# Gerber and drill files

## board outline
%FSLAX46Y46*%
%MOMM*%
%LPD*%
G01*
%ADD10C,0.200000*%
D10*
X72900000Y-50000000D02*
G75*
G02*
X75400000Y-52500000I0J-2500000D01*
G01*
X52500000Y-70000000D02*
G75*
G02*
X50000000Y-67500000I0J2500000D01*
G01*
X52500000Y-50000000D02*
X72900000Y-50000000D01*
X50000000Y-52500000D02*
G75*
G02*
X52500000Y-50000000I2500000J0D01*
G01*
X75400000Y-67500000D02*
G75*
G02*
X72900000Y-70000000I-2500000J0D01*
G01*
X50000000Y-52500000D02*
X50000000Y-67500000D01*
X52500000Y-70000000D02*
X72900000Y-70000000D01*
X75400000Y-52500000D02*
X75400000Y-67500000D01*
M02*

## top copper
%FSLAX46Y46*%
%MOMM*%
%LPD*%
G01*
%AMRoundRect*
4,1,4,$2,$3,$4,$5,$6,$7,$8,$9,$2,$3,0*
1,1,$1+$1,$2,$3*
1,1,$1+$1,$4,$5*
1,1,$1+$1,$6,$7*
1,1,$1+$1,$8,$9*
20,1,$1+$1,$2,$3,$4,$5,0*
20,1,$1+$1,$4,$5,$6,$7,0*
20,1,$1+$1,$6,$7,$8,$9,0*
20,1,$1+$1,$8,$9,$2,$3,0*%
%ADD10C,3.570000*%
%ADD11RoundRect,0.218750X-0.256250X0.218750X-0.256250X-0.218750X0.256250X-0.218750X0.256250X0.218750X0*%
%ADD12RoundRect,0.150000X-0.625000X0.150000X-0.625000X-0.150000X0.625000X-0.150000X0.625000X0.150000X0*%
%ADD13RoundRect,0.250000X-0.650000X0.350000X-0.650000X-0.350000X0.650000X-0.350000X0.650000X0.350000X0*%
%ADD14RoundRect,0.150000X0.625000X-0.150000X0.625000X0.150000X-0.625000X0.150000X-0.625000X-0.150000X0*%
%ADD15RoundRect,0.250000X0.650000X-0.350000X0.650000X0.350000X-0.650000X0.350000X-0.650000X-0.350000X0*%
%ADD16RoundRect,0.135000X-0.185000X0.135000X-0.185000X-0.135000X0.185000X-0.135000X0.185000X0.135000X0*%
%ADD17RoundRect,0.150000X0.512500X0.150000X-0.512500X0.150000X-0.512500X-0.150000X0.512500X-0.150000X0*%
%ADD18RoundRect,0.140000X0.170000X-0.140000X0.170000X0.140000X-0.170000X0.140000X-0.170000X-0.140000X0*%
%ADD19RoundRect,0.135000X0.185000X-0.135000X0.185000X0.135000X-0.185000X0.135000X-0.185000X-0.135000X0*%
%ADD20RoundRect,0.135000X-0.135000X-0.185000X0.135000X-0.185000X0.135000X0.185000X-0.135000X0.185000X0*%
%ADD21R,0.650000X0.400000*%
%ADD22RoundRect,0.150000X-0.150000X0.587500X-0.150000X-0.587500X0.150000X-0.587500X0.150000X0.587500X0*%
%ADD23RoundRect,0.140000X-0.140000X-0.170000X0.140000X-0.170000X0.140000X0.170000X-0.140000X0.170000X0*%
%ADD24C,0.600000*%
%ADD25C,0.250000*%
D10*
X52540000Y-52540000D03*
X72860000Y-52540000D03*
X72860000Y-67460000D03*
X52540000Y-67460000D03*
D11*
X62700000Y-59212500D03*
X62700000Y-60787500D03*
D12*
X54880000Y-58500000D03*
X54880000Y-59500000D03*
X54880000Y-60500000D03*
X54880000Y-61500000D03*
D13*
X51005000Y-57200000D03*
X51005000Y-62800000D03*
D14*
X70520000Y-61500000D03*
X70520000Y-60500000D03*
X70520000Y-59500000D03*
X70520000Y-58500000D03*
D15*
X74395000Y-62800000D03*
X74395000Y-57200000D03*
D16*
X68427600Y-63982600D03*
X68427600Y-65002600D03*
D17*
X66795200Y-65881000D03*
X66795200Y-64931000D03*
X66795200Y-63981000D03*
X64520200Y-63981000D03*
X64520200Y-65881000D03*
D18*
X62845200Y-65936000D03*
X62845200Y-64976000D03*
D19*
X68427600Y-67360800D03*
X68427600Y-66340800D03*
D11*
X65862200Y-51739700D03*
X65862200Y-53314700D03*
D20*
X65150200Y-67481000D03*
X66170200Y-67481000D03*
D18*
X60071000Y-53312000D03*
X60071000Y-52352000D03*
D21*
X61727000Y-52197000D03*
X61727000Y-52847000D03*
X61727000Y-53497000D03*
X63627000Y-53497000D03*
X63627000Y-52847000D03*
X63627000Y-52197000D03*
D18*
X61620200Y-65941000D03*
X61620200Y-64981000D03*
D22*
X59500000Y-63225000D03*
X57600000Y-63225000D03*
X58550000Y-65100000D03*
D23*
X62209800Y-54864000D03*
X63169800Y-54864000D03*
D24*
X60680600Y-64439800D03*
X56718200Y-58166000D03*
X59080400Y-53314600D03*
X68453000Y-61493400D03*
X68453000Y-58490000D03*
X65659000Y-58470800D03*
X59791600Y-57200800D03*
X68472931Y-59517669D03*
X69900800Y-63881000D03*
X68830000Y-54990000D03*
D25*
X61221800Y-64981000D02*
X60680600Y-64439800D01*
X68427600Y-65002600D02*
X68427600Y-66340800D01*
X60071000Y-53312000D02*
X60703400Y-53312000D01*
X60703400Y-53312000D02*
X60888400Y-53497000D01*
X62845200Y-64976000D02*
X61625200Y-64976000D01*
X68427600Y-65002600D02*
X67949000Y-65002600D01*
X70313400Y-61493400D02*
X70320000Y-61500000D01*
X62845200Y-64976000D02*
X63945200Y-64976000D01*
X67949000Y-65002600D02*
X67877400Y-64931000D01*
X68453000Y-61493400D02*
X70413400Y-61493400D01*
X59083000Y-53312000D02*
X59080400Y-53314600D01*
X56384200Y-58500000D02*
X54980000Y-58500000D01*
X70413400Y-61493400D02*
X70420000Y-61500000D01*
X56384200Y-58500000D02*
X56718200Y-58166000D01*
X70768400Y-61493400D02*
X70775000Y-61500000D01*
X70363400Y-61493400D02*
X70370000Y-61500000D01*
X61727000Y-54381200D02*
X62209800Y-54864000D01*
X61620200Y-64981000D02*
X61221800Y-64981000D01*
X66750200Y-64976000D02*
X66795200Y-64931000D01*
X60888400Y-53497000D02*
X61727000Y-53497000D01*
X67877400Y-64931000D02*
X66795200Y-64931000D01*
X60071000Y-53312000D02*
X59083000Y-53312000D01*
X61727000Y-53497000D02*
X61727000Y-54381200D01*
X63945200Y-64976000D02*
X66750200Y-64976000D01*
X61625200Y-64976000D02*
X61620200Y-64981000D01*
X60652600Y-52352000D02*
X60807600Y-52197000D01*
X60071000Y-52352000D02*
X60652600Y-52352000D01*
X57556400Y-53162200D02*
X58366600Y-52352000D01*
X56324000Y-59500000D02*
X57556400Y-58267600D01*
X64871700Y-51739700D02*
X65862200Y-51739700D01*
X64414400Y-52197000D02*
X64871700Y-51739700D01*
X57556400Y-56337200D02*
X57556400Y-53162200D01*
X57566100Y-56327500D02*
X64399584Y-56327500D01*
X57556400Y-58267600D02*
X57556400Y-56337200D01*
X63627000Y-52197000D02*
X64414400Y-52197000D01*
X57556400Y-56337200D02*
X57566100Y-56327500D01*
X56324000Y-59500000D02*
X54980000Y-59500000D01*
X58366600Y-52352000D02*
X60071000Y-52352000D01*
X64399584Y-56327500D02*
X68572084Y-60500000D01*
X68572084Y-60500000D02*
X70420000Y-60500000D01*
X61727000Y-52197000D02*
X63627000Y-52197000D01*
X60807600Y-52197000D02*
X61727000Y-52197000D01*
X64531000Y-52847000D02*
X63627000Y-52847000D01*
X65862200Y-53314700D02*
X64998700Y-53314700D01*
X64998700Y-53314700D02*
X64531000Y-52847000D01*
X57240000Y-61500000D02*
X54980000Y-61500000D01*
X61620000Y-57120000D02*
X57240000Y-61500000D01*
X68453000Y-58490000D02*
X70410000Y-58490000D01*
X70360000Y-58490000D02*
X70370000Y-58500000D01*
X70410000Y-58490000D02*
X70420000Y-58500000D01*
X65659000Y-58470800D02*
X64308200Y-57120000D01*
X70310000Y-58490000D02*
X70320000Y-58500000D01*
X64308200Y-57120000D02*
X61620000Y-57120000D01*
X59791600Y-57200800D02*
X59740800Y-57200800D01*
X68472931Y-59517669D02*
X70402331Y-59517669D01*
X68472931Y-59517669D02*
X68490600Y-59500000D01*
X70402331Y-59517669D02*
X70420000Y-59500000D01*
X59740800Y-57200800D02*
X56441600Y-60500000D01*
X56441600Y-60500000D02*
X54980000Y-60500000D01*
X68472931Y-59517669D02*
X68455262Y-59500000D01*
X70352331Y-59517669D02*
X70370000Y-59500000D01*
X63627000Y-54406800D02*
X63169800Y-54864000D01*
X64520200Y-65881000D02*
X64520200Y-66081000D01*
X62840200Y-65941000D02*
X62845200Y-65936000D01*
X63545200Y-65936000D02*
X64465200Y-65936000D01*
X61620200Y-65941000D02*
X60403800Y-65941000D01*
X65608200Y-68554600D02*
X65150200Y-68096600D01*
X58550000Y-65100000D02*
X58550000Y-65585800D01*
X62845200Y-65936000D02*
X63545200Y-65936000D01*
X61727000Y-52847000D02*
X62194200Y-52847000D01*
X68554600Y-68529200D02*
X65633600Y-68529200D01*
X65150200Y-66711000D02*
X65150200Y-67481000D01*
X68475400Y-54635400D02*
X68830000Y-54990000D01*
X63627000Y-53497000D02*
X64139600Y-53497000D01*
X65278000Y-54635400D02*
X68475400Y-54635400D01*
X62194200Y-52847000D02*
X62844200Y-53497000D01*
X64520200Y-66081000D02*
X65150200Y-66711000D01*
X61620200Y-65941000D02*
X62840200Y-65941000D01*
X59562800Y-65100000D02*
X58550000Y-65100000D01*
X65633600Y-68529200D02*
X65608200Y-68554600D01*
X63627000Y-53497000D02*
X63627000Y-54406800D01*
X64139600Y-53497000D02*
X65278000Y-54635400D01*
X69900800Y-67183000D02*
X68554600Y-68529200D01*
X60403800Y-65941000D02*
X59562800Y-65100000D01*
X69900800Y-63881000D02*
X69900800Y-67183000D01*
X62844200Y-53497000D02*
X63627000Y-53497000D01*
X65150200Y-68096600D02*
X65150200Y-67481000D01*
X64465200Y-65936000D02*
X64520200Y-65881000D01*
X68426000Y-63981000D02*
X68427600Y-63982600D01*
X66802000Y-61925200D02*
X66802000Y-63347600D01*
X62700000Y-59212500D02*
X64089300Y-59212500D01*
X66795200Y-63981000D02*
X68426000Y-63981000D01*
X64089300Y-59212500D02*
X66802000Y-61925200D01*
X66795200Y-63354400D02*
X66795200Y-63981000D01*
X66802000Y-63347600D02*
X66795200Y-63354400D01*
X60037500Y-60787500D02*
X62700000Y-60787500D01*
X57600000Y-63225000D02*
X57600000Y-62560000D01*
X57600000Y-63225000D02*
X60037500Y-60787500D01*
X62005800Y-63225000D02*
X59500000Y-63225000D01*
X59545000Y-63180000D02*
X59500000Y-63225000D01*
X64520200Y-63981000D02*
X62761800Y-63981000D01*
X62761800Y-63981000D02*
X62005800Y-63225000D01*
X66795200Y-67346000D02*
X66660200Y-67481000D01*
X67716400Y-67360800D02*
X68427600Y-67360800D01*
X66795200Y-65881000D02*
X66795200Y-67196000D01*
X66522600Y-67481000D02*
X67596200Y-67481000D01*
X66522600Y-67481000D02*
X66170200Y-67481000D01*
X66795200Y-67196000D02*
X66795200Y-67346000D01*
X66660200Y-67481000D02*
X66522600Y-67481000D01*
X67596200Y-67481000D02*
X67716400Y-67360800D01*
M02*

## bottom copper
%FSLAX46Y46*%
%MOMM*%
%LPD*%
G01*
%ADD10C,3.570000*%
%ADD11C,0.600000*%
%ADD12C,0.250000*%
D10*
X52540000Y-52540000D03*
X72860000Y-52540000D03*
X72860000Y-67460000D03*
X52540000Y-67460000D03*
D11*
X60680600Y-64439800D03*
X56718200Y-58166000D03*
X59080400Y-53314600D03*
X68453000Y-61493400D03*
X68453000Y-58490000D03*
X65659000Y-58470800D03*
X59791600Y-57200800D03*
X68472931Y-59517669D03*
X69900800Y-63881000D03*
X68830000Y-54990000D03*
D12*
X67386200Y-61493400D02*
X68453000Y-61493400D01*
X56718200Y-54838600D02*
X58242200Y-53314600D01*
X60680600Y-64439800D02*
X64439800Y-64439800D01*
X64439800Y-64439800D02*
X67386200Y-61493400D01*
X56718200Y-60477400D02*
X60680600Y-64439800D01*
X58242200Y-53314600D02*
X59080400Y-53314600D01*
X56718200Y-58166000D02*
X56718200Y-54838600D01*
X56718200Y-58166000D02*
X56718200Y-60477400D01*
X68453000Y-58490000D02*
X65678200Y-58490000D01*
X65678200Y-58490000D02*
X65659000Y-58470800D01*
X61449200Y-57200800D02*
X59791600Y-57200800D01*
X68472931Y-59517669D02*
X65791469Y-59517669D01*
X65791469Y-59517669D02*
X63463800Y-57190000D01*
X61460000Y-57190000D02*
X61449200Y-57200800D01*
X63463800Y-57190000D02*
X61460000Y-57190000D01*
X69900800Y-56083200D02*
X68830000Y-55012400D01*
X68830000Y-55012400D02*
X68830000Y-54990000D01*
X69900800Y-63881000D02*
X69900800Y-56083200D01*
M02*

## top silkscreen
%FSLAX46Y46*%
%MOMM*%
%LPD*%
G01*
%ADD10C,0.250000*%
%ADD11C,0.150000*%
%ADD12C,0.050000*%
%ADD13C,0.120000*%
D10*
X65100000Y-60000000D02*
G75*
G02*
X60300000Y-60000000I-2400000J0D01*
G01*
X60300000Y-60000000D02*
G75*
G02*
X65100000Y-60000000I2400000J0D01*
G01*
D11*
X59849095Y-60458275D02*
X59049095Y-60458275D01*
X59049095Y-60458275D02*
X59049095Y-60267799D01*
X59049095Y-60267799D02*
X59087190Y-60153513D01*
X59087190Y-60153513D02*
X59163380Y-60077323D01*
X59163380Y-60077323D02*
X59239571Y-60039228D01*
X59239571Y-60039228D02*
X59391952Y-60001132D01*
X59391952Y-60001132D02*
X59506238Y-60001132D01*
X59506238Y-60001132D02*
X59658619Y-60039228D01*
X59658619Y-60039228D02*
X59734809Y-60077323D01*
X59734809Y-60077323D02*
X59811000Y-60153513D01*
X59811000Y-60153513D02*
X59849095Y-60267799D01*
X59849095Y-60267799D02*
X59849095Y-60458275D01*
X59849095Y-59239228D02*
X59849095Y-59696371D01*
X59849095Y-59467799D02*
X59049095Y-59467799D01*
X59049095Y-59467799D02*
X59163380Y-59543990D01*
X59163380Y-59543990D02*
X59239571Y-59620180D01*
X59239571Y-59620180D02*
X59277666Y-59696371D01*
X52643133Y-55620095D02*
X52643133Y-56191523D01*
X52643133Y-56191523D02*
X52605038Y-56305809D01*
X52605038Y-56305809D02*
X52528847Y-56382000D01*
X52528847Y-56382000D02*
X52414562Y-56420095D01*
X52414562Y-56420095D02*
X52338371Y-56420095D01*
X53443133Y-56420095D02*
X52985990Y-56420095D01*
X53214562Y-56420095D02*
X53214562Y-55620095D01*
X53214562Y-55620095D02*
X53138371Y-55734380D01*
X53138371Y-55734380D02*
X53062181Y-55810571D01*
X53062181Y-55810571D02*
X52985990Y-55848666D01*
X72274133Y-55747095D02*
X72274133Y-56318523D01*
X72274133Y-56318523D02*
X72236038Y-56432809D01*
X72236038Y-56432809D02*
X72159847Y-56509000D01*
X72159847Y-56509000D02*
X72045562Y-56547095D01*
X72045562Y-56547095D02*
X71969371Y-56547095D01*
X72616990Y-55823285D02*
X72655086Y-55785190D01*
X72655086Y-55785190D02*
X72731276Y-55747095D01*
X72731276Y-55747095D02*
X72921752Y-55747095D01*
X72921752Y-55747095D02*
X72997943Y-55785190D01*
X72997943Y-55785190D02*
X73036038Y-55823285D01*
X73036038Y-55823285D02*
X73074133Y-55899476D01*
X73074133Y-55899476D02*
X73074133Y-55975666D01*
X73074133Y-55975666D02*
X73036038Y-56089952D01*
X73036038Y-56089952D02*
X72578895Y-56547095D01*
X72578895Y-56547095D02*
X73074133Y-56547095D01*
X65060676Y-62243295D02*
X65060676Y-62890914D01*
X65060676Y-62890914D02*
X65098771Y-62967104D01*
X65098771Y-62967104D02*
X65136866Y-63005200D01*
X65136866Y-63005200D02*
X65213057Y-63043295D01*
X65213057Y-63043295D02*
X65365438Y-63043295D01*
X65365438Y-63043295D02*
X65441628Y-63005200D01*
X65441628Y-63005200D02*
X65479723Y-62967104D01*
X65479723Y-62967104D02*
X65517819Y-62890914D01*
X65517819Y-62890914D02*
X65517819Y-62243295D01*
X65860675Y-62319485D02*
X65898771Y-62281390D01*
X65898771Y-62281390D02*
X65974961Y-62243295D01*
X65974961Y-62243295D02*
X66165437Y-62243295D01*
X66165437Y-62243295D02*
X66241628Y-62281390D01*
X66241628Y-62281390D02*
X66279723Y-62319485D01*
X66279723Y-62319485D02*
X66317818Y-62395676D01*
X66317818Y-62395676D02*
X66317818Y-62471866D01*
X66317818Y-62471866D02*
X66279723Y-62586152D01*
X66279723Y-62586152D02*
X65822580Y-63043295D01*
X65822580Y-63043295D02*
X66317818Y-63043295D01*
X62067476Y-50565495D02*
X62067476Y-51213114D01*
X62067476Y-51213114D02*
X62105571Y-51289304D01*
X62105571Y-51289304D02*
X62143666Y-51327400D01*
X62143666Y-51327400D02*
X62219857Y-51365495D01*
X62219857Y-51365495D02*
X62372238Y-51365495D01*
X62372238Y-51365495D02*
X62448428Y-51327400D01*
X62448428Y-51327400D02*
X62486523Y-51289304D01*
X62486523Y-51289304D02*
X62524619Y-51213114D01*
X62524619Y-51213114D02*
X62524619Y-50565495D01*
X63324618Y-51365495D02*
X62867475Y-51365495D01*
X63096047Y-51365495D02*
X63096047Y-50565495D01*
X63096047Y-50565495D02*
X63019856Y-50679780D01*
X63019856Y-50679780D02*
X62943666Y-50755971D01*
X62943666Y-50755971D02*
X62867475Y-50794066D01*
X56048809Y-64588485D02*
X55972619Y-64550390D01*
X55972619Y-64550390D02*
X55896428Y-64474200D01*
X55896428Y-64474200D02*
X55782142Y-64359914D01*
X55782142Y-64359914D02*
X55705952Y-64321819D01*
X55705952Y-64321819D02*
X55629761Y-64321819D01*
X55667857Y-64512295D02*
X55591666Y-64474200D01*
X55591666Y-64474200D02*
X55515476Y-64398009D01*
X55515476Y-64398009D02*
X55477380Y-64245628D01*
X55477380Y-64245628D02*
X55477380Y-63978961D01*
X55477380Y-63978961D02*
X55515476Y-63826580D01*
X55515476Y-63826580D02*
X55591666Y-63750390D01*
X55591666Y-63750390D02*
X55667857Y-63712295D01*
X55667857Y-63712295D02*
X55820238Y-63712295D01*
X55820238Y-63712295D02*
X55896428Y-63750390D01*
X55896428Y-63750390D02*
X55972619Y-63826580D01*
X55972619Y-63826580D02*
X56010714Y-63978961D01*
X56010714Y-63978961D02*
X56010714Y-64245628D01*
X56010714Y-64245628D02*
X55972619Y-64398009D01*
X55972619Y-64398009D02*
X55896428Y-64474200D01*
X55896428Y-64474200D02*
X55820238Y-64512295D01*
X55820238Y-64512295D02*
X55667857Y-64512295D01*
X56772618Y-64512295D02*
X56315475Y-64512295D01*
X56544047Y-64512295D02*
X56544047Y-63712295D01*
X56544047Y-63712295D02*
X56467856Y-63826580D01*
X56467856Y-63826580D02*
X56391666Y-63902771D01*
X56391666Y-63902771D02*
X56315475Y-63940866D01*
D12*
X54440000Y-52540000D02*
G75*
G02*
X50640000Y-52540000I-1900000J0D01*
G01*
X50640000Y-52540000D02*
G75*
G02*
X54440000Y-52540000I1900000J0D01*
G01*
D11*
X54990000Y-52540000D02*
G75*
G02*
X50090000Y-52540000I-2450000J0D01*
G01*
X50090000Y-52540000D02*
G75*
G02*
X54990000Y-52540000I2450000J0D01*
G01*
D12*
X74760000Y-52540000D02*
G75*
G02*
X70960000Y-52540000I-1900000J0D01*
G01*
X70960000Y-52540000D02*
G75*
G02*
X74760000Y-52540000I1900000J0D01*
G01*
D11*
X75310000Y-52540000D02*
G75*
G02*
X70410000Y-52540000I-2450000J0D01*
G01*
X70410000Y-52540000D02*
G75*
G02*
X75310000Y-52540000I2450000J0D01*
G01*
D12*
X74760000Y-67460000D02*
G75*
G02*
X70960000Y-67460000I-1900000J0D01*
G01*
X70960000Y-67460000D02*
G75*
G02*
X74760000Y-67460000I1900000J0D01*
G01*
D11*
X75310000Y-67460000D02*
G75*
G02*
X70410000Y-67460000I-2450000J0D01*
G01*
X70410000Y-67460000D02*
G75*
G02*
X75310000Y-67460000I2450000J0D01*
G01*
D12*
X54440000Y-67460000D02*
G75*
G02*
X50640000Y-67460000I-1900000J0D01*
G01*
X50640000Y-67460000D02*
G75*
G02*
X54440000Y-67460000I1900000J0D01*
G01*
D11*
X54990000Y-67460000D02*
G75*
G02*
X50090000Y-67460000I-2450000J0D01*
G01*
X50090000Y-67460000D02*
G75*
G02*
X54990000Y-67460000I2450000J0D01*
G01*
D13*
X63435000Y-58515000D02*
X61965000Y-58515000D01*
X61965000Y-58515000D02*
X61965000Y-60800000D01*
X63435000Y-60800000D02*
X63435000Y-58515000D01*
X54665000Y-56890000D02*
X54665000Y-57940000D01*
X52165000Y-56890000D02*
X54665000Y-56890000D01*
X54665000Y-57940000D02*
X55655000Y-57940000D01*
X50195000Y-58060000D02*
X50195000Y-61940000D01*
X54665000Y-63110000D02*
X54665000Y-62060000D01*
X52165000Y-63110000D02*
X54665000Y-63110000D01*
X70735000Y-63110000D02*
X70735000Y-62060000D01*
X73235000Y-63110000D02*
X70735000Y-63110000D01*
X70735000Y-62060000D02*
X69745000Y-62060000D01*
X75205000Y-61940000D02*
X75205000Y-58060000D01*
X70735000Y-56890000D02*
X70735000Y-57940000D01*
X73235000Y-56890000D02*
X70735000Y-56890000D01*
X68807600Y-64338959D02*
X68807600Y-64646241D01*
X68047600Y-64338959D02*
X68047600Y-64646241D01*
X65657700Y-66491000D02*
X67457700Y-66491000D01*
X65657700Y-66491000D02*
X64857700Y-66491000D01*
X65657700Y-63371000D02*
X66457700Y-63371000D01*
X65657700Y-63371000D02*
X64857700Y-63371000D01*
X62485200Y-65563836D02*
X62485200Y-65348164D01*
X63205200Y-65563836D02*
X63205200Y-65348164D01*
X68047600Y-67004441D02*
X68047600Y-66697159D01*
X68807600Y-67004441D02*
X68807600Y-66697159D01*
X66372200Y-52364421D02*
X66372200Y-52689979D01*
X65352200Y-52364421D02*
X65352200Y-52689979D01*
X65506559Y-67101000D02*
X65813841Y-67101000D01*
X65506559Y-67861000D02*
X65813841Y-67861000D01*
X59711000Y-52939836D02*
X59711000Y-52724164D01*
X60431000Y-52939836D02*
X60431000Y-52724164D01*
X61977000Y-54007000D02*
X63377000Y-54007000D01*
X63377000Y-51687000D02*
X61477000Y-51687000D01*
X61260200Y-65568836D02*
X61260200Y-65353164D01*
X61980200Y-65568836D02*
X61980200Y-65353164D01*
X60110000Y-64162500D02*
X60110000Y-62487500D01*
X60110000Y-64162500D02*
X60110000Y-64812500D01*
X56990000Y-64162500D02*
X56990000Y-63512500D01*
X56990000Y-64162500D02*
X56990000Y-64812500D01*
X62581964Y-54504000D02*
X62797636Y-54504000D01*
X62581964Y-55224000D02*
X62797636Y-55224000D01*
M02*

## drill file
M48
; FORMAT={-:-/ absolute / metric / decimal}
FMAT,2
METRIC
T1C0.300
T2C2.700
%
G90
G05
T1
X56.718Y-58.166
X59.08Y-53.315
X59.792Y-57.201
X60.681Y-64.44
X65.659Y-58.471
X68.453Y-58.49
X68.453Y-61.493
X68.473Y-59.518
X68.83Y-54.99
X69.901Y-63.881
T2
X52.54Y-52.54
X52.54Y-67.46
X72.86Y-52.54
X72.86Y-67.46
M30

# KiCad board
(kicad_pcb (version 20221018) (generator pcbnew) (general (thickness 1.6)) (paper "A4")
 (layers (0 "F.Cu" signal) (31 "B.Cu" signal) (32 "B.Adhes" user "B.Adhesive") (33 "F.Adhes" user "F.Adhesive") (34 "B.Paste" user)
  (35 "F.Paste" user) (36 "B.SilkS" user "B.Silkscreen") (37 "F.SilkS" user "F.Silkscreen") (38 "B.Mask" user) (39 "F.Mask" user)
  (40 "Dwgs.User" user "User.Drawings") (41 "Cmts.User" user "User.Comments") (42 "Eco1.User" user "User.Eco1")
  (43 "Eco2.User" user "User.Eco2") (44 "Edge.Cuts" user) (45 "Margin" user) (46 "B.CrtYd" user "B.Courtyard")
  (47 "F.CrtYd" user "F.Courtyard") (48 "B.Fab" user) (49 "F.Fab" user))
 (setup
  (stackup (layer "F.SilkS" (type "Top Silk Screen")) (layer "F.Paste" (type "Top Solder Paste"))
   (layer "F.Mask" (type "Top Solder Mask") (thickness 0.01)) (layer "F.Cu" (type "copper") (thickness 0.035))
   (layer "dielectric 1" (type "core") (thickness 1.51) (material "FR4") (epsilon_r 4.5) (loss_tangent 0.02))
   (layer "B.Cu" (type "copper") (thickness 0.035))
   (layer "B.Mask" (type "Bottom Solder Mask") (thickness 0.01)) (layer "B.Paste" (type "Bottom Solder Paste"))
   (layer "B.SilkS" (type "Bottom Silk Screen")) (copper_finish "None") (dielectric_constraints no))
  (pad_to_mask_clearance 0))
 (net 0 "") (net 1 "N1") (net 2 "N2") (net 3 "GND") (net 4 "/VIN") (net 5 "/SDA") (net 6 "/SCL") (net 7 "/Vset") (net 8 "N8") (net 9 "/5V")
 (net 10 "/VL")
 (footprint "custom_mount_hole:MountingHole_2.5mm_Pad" (layer "F.Cu") (at 52.54 52.54)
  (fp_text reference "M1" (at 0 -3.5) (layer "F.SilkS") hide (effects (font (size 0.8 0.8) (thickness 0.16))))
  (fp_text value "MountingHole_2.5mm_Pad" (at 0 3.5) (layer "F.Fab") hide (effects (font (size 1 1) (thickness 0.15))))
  (fp_circle (center 0 0) (end 1.9 0) (stroke (width 0.05) (type solid)) (fill none) (layer "F.SilkS"))
  (fp_circle (center 0 0) (end 2.45 0) (stroke (width 0.15) (type solid)) (fill none) (layer "F.SilkS"))
  (pad "~" thru_hole circle (at 0 0) (size 3.57 3.57) (drill 2.7) (layers "*.Cu" "*.Mask")))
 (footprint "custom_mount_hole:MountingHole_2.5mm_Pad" (layer "F.Cu") (at 72.86 52.54)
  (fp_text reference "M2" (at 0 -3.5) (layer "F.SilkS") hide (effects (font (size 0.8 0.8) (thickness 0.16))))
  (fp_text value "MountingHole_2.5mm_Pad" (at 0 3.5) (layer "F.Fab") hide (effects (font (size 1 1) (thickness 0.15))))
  (fp_circle (center 0 0) (end 1.9 0) (stroke (width 0.05) (type solid)) (fill none) (layer "F.SilkS"))
  (fp_circle (center 0 0) (end 2.45 0) (stroke (width 0.15) (type solid)) (fill none) (layer "F.SilkS"))
  (pad "~" thru_hole circle (at 0 0) (size 3.57 3.57) (drill 2.7) (layers "*.Cu" "*.Mask")))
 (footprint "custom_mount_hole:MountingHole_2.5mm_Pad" (layer "F.Cu") (at 72.86 67.46)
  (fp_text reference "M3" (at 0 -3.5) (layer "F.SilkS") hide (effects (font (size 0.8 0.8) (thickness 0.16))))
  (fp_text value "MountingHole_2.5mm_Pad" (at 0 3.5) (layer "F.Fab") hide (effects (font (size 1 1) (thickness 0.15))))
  (fp_circle (center 0 0) (end 1.9 0) (stroke (width 0.05) (type solid)) (fill none) (layer "F.SilkS"))
  (fp_circle (center 0 0) (end 2.45 0) (stroke (width 0.15) (type solid)) (fill none) (layer "F.SilkS"))
  (pad "~" thru_hole circle (at 0 0) (size 3.57 3.57) (drill 2.7) (layers "*.Cu" "*.Mask")))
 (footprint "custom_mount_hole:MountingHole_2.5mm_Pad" (layer "F.Cu") (at 52.54 67.46)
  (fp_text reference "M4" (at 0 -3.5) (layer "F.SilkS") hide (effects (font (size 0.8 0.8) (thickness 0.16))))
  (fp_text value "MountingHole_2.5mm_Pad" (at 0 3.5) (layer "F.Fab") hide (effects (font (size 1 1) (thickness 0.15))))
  (fp_circle (center 0 0) (end 1.9 0) (stroke (width 0.05) (type solid)) (fill none) (layer "F.SilkS"))
  (fp_circle (center 0 0) (end 2.45 0) (stroke (width 0.15) (type solid)) (fill none) (layer "F.SilkS"))
  (pad "~" thru_hole circle (at 0 0) (size 3.57 3.57) (drill 2.7) (layers "*.Cu" "*.Mask")))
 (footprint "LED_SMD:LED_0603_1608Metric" (layer "F.Cu") (at 62.7 60 -90)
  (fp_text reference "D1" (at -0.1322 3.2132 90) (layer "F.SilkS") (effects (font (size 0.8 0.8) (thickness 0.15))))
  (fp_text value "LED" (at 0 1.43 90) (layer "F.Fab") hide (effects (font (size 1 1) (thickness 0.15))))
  (fp_line (start -1.485 -0.735) (end -1.485 0.735) (stroke (width 0.12) (type solid)) (layer "F.SilkS"))
  (fp_line (start -1.485 0.735) (end 0.8 0.735) (stroke (width 0.12) (type solid)) (layer "F.SilkS"))
  (fp_line (start 0.8 -0.735) (end -1.485 -0.735) (stroke (width 0.12) (type solid)) (layer "F.SilkS"))
  (pad "1" smd roundrect (at -0.7875 0 270) (size 0.875 0.95) (layers "F.Cu" "F.Paste" "F.Mask") (roundrect_rratio 0.25) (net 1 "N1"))
  (pad "2" smd roundrect (at 0.7875 0 270) (size 0.875 0.95) (layers "F.Cu" "F.Paste" "F.Mask") (roundrect_rratio 0.25) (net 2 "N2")))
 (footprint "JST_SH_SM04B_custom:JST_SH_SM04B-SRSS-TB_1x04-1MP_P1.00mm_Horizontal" (layer "F.Cu") (at 52.88 60 -90)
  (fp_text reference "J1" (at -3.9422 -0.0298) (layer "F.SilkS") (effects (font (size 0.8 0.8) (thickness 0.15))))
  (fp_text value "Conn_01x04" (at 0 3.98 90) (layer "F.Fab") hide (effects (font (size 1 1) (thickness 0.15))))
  (fp_line (start -3.11 -1.785) (end -2.06 -1.785) (stroke (width 0.12) (type solid)) (layer "F.SilkS"))
  (fp_line (start -3.11 0.715) (end -3.11 -1.785) (stroke (width 0.12) (type solid)) (layer "F.SilkS"))
  (fp_line (start -2.06 -1.785) (end -2.06 -2.775) (stroke (width 0.12) (type solid)) (layer "F.SilkS"))
  (fp_line (start -1.94 2.685) (end 1.94 2.685) (stroke (width 0.12) (type solid)) (layer "F.SilkS"))
  (fp_line (start 3.11 -1.785) (end 2.06 -1.785) (stroke (width 0.12) (type solid)) (layer "F.SilkS"))
  (fp_line (start 3.11 0.715) (end 3.11 -1.785) (stroke (width 0.12) (type solid)) (layer "F.SilkS"))
  (pad "1" smd roundrect (at -1.5 -2 270) (size 0.6 1.55) (layers "F.Cu" "F.Paste" "F.Mask") (roundrect_rratio 0.25) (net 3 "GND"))
  (pad "2" smd roundrect (at -0.5 -2 270) (size 0.6 1.55) (layers "F.Cu" "F.Paste" "F.Mask") (roundrect_rratio 0.25) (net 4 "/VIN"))
  (pad "3" smd roundrect (at 0.5 -2 270) (size 0.6 1.55) (layers "F.Cu" "F.Paste" "F.Mask") (roundrect_rratio 0.25) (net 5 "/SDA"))
  (pad "4" smd roundrect (at 1.5 -2 270) (size 0.6 1.55) (layers "F.Cu" "F.Paste" "F.Mask") (roundrect_rratio 0.25) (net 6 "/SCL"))
  (pad "MP" smd roundrect (at -2.8 1.875 270) (size 1.2 1.8) (layers "F.Cu" "F.Paste" "F.Mask") (roundrect_rratio 0.2083333333))
  (pad "MP" smd roundrect (at 2.8 1.875 270) (size 1.2 1.8) (layers "F.Cu" "F.Paste" "F.Mask") (roundrect_rratio 0.2083333333)))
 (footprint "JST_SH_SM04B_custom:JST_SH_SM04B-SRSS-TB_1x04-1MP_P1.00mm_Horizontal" (layer "F.Cu") (at 72.52 60 90)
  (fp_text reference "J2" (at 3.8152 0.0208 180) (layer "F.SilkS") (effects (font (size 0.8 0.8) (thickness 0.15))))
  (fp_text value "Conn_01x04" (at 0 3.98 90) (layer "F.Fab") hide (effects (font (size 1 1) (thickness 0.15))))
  (fp_line (start -3.11 -1.785) (end -2.06 -1.785) (stroke (width 0.12) (type solid)) (layer "F.SilkS"))
  (fp_line (start -3.11 0.715) (end -3.11 -1.785) (stroke (width 0.12) (type solid)) (layer "F.SilkS"))
  (fp_line (start -2.06 -1.785) (end -2.06 -2.775) (stroke (width 0.12) (type solid)) (layer "F.SilkS"))
  (fp_line (start -1.94 2.685) (end 1.94 2.685) (stroke (width 0.12) (type solid)) (layer "F.SilkS"))
  (fp_line (start 3.11 -1.785) (end 2.06 -1.785) (stroke (width 0.12) (type solid)) (layer "F.SilkS"))
  (fp_line (start 3.11 0.715) (end 3.11 -1.785) (stroke (width 0.12) (type solid)) (layer "F.SilkS"))
  (pad "1" smd roundrect (at -1.5 -2 90) (size 0.6 1.55) (layers "F.Cu" "F.Paste" "F.Mask") (roundrect_rratio 0.25) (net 3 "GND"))
  (pad "2" smd roundrect (at -0.5 -2 90) (size 0.6 1.55) (layers "F.Cu" "F.Paste" "F.Mask") (roundrect_rratio 0.25) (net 4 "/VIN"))
  (pad "3" smd roundrect (at 0.5 -2 90) (size 0.6 1.55) (layers "F.Cu" "F.Paste" "F.Mask") (roundrect_rratio 0.25) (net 5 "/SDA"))
  (pad "4" smd roundrect (at 1.5 -2 90) (size 0.6 1.55) (layers "F.Cu" "F.Paste" "F.Mask") (roundrect_rratio 0.25) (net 6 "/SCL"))
  (pad "MP" smd roundrect (at -2.8 1.875 90) (size 1.2 1.8) (layers "F.Cu" "F.Paste" "F.Mask") (roundrect_rratio 0.2083333333))
  (pad "MP" smd roundrect (at 2.8 1.875 90) (size 1.2 1.8) (layers "F.Cu" "F.Paste" "F.Mask") (roundrect_rratio 0.2083333333)))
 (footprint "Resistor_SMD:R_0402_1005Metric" (layer "F.Cu") (at 68.4276 64.4926 -90)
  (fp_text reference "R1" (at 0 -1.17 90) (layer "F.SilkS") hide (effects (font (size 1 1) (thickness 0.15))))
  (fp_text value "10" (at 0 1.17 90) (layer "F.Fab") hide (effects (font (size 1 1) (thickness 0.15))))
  (fp_line (start -0.153641 -0.38) (end 0.153641 -0.38) (stroke (width 0.12) (type solid)) (layer "F.SilkS"))
  (fp_line (start -0.153641 0.38) (end 0.153641 0.38) (stroke (width 0.12) (type solid)) (layer "F.SilkS"))
  (pad "1" smd roundrect (at -0.51 0 270) (size 0.54 0.64) (layers "F.Cu" "F.Paste" "F.Mask") (roundrect_rratio 0.25) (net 1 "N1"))
  (pad "2" smd roundrect (at 0.51 0 270) (size 0.54 0.64) (layers "F.Cu" "F.Paste" "F.Mask") (roundrect_rratio 0.25) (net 3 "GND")))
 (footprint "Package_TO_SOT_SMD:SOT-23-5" (layer "F.Cu") (at 65.6577 64.931 180)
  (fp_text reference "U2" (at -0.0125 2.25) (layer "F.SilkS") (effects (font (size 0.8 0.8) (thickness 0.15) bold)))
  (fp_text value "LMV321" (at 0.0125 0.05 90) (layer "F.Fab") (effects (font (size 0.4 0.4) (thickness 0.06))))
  (fp_line (start 0 -1.56) (end -1.8 -1.56) (stroke (width 0.12) (type solid)) (layer "F.SilkS"))
  (fp_line (start 0 -1.56) (end 0.8 -1.56) (stroke (width 0.12) (type solid)) (layer "F.SilkS"))
  (fp_line (start 0 1.56) (end -0.8 1.56) (stroke (width 0.12) (type solid)) (layer "F.SilkS"))
  (fp_line (start 0 1.56) (end 0.8 1.56) (stroke (width 0.12) (type solid)) (layer "F.SilkS"))
  (pad "1" smd roundrect (at -1.1375 -0.95 180) (size 1.325 0.6) (layers "F.Cu" "F.Paste" "F.Mask") (roundrect_rratio 0.25) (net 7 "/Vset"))
  (pad "2" smd roundrect (at -1.1375 0 180) (size 1.325 0.6) (layers "F.Cu" "F.Paste" "F.Mask") (roundrect_rratio 0.25) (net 3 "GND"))
  (pad "3" smd roundrect (at -1.1375 0.95 180) (size 1.325 0.6) (layers "F.Cu" "F.Paste" "F.Mask") (roundrect_rratio 0.25) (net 1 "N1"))
  (pad "4" smd roundrect (at 1.1375 0.95 180) (size 1.325 0.6) (layers "F.Cu" "F.Paste" "F.Mask") (roundrect_rratio 0.25) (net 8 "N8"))
  (pad "5" smd roundrect (at 1.1375 -0.95 180) (size 1.325 0.6) (layers "F.Cu" "F.Paste" "F.Mask") (roundrect_rratio 0.25) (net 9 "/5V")))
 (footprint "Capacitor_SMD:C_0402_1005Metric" (layer "F.Cu") (at 62.8452 65.456 90)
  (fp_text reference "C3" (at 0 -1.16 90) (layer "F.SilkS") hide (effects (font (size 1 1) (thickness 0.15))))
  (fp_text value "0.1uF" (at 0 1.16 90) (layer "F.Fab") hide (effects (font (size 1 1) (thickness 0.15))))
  (fp_line (start -0.107836 -0.36) (end 0.107836 -0.36) (stroke (width 0.12) (type solid)) (layer "F.SilkS"))
  (fp_line (start -0.107836 0.36) (end 0.107836 0.36) (stroke (width 0.12) (type solid)) (layer "F.SilkS"))
  (pad "1" smd roundrect (at -0.48 0 90) (size 0.56 0.62) (layers "F.Cu" "F.Paste" "F.Mask") (roundrect_rratio 0.25) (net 9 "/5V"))
  (pad "2" smd roundrect (at 0.48 0 90) (size 0.56 0.62) (layers "F.Cu" "F.Paste" "F.Mask") (roundrect_rratio 0.25) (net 3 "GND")))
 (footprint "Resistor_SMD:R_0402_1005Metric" (layer "F.Cu") (at 68.4276 66.8508 90)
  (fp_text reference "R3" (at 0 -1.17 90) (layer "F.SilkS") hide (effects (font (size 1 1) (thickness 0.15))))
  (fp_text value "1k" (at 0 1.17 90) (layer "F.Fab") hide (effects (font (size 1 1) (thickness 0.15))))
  (fp_line (start -0.153641 -0.38) (end 0.153641 -0.38) (stroke (width 0.12) (type solid)) (layer "F.SilkS"))
  (fp_line (start -0.153641 0.38) (end 0.153641 0.38) (stroke (width 0.12) (type solid)) (layer "F.SilkS"))
  (pad "1" smd roundrect (at -0.51 0 90) (size 0.54 0.64) (layers "F.Cu" "F.Paste" "F.Mask") (roundrect_rratio 0.25) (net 7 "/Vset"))
  (pad "2" smd roundrect (at 0.51 0 90) (size 0.54 0.64) (layers "F.Cu" "F.Paste" "F.Mask") (roundrect_rratio 0.25) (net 3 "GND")))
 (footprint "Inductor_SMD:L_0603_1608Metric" (layer "F.Cu") (at 65.8622 52.5272 -90)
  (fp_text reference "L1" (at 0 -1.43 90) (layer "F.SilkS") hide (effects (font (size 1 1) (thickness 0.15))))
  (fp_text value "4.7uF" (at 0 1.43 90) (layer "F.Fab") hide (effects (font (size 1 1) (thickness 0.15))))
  (fp_line (start -0.162779 -0.51) (end 0.162779 -0.51) (stroke (width 0.12) (type solid)) (layer "F.SilkS"))
  (fp_line (start -0.162779 0.51) (end 0.162779 0.51) (stroke (width 0.12) (type solid)) (layer "F.SilkS"))
  (pad "1" smd roundrect (at -0.7875 0 270) (size 0.875 0.95) (layers "F.Cu" "F.Paste" "F.Mask") (roundrect_rratio 0.25) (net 4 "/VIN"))
  (pad "2" smd roundrect (at 0.7875 0 270) (size 0.875 0.95) (layers "F.Cu" "F.Paste" "F.Mask") (roundrect_rratio 0.25) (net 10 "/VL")))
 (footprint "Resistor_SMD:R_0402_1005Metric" (layer "F.Cu") (at 65.6602 67.481)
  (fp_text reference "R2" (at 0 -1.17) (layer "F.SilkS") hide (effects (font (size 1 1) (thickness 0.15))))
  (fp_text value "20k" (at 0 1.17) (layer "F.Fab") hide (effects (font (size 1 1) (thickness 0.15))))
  (fp_line (start -0.153641 -0.38) (end 0.153641 -0.38) (stroke (width 0.12) (type solid)) (layer "F.SilkS"))
  (fp_line (start -0.153641 0.38) (end 0.153641 0.38) (stroke (width 0.12) (type solid)) (layer "F.SilkS"))
  (pad "1" smd roundrect (at -0.51 0) (size 0.54 0.64) (layers "F.Cu" "F.Paste" "F.Mask") (roundrect_rratio 0.25) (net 9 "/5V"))
  (pad "2" smd roundrect (at 0.51 0) (size 0.54 0.64) (layers "F.Cu" "F.Paste" "F.Mask") (roundrect_rratio 0.25) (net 7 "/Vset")))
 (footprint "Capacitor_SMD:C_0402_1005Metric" (layer "F.Cu") (at 60.071 52.832 90)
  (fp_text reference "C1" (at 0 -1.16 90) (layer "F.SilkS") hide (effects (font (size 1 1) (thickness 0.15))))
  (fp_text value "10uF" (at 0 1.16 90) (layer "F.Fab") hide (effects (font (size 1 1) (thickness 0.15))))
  (fp_line (start -0.107836 -0.36) (end 0.107836 -0.36) (stroke (width 0.12) (type solid)) (layer "F.SilkS"))
  (fp_line (start -0.107836 0.36) (end 0.107836 0.36) (stroke (width 0.12) (type solid)) (layer "F.SilkS"))
  (pad "1" smd roundrect (at -0.48 0 90) (size 0.56 0.62) (layers "F.Cu" "F.Paste" "F.Mask") (roundrect_rratio 0.25) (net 3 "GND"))
  (pad "2" smd roundrect (at 0.48 0 90) (size 0.56 0.62) (layers "F.Cu" "F.Paste" "F.Mask") (roundrect_rratio 0.25) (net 4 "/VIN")))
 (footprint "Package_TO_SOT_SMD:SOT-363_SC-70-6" (layer "F.Cu") (at 62.677 52.847)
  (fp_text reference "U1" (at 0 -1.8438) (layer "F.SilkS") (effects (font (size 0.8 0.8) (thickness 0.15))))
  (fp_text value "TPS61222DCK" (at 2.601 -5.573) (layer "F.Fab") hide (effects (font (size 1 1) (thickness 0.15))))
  (fp_line (start -0.7 1.16) (end 0.7 1.16) (stroke (width 0.12) (type solid)) (layer "F.SilkS"))
  (fp_line (start 0.7 -1.16) (end -1.2 -1.16) (stroke (width 0.12) (type solid)) (layer "F.SilkS"))
  (pad "1" smd rect (at -0.95 -0.65) (size 0.65 0.4) (layers "F.Cu" "F.Paste" "F.Mask") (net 4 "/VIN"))
  (pad "2" smd rect (at -0.95 0) (size 0.65 0.4) (layers "F.Cu" "F.Paste" "F.Mask") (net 9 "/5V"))
  (pad "3" smd rect (at -0.95 0.65) (size 0.65 0.4) (layers "F.Cu" "F.Paste" "F.Mask") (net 3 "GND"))
  (pad "4" smd rect (at 0.95 0.65) (size 0.65 0.4) (layers "F.Cu" "F.Paste" "F.Mask") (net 9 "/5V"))
  (pad "5" smd rect (at 0.95 0) (size 0.65 0.4) (layers "F.Cu" "F.Paste" "F.Mask") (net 10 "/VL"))
  (pad "6" smd rect (at 0.95 -0.65) (size 0.65 0.4) (layers "F.Cu" "F.Paste" "F.Mask") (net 4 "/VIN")))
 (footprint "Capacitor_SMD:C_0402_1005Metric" (layer "F.Cu") (at 61.6202 65.461 90)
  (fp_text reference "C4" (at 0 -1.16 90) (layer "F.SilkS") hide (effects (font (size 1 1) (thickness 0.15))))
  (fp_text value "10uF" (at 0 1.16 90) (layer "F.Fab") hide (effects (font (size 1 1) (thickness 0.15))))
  (fp_line (start -0.107836 -0.36) (end 0.107836 -0.36) (stroke (width 0.12) (type solid)) (layer "F.SilkS"))
  (fp_line (start -0.107836 0.36) (end 0.107836 0.36) (stroke (width 0.12) (type solid)) (layer "F.SilkS"))
  (pad "1" smd roundrect (at -0.48 0 90) (size 0.56 0.62) (layers "F.Cu" "F.Paste" "F.Mask") (roundrect_rratio 0.25) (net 9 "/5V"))
  (pad "2" smd roundrect (at 0.48 0 90) (size 0.56 0.62) (layers "F.Cu" "F.Paste" "F.Mask") (roundrect_rratio 0.25) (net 3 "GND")))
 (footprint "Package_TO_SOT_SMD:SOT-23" (layer "F.Cu") (at 58.55 64.1625 -90)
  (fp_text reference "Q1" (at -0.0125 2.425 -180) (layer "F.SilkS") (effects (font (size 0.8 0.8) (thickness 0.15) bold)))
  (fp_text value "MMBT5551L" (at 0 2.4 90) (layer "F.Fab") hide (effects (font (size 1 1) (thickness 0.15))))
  (fp_line (start 0 -1.56) (end -1.675 -1.56) (stroke (width 0.12) (type solid)) (layer "F.SilkS"))
  (fp_line (start 0 -1.56) (end 0.65 -1.56) (stroke (width 0.12) (type solid)) (layer "F.SilkS"))
  (fp_line (start 0 1.56) (end -0.65 1.56) (stroke (width 0.12) (type solid)) (layer "F.SilkS"))
  (fp_line (start 0 1.56) (end 0.65 1.56) (stroke (width 0.12) (type solid)) (layer "F.SilkS"))
  (pad "1" smd roundrect (at -0.9375 -0.95 270) (size 1.475 0.6) (layers "F.Cu" "F.Paste" "F.Mask") (roundrect_rratio 0.25) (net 8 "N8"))
  (pad "2" smd roundrect (at -0.9375 0.95 270) (size 1.475 0.6) (layers "F.Cu" "F.Paste" "F.Mask") (roundrect_rratio 0.25) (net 2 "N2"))
  (pad "3" smd roundrect (at 0.9375 0 270) (size 1.475 0.6) (layers "F.Cu" "F.Paste" "F.Mask") (roundrect_rratio 0.25) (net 9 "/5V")))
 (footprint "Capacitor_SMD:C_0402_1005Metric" (layer "F.Cu") (at 62.6898 54.864)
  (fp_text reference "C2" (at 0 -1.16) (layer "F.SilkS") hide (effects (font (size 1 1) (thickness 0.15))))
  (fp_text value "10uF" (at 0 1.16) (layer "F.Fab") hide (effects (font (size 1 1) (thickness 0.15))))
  (fp_line (start -0.107836 -0.36) (end 0.107836 -0.36) (stroke (width 0.12) (type solid)) (layer "F.SilkS"))
  (fp_line (start -0.107836 0.36) (end 0.107836 0.36) (stroke (width 0.12) (type solid)) (layer "F.SilkS"))
  (pad "1" smd roundrect (at -0.48 0) (size 0.56 0.62) (layers "F.Cu" "F.Paste" "F.Mask") (roundrect_rratio 0.25) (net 3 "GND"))
  (pad "2" smd roundrect (at 0.48 0) (size 0.56 0.62) (layers "F.Cu" "F.Paste" "F.Mask") (roundrect_rratio 0.25) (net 9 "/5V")))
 (gr_circle (center 62.7 60) (end 65.1 60) (stroke (width 0.25) (type solid)) (fill none) (layer "F.SilkS"))
 (gr_arc (start 72.9 50) (mid 74.667767 50.732233) (end 75.4 52.5) (stroke (width 0.2) (type solid)) (layer "Edge.Cuts"))
 (gr_arc (start 52.5 70) (mid 50.732233 69.267767) (end 50 67.5) (stroke (width 0.2) (type solid)) (layer "Edge.Cuts"))
 (gr_line (start 52.5 50) (end 72.9 50) (stroke (width 0.2) (type solid)) (layer "Edge.Cuts"))
 (gr_arc (start 50 52.5) (mid 50.732233 50.732233) (end 52.5 50) (stroke (width 0.2) (type solid)) (layer "Edge.Cuts"))
 (gr_arc (start 75.4 67.5) (mid 74.667767 69.267767) (end 72.9 70) (stroke (width 0.2) (type solid)) (layer "Edge.Cuts"))
 (gr_line (start 50 52.5) (end 50 67.5) (stroke (width 0.2) (type solid)) (layer "Edge.Cuts"))
 (gr_line (start 52.5 70) (end 72.9 70) (stroke (width 0.2) (type solid)) (layer "Edge.Cuts"))
 (gr_line (start 75.4 52.5) (end 75.4 67.5) (stroke (width 0.2) (type solid)) (layer "Edge.Cuts"))
 (segment (start 61.2218 64.981) (end 60.6806 64.4398) (width 0.25) (layer "F.Cu") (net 3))
 (segment (start 68.4276 65.0026) (end 68.4276 66.3408) (width 0.25) (layer "F.Cu") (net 3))
 (segment (start 60.071 53.312) (end 60.7034 53.312) (width 0.25) (layer "F.Cu") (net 3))
 (segment (start 60.7034 53.312) (end 60.8884 53.497) (width 0.25) (layer "F.Cu") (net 3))
 (segment (start 62.8452 64.976) (end 61.6252 64.976) (width 0.25) (layer "F.Cu") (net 3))
 (segment (start 68.4276 65.0026) (end 67.949 65.0026) (width 0.25) (layer "F.Cu") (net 3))
 (segment (start 70.3134 61.4934) (end 70.32 61.5) (width 0.25) (layer "F.Cu") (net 3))
 (segment (start 62.8452 64.976) (end 63.9452 64.976) (width 0.25) (layer "F.Cu") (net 3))
 (segment (start 67.949 65.0026) (end 67.8774 64.931) (width 0.25) (layer "F.Cu") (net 3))
 (segment (start 68.453 61.4934) (end 70.4134 61.4934) (width 0.25) (layer "F.Cu") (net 3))
 (segment (start 59.083 53.312) (end 59.0804 53.3146) (width 0.25) (layer "F.Cu") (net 3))
 (segment (start 56.3842 58.5) (end 54.98 58.5) (width 0.25) (layer "F.Cu") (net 3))
 (segment (start 70.4134 61.4934) (end 70.42 61.5) (width 0.25) (layer "F.Cu") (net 3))
 (segment (start 56.3842 58.5) (end 56.7182 58.166) (width 0.25) (layer "F.Cu") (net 3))
 (segment (start 70.7684 61.4934) (end 70.775 61.5) (width 0.25) (layer "F.Cu") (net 3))
 (segment (start 70.3634 61.4934) (end 70.37 61.5) (width 0.25) (layer "F.Cu") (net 3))
 (segment (start 61.727 54.3812) (end 62.2098 54.864) (width 0.25) (layer "F.Cu") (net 3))
 (segment (start 61.6202 64.981) (end 61.2218 64.981) (width 0.25) (layer "F.Cu") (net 3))
 (segment (start 66.7502 64.976) (end 66.7952 64.931) (width 0.25) (layer "F.Cu") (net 3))
 (segment (start 60.8884 53.497) (end 61.727 53.497) (width 0.25) (layer "F.Cu") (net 3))
 (segment (start 67.8774 64.931) (end 66.7952 64.931) (width 0.25) (layer "F.Cu") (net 3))
 (segment (start 60.071 53.312) (end 59.083 53.312) (width 0.25) (layer "F.Cu") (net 3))
 (segment (start 61.727 53.497) (end 61.727 54.3812) (width 0.25) (layer "F.Cu") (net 3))
 (segment (start 63.9452 64.976) (end 66.7502 64.976) (width 0.25) (layer "F.Cu") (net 3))
 (segment (start 61.6252 64.976) (end 61.6202 64.981) (width 0.25) (layer "F.Cu") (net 3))
 (via (at 60.6806 64.4398) (size 0.6) (drill 0.3) (layers "F.Cu" "B.Cu") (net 3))
 (via (at 56.7182 58.166) (size 0.6) (drill 0.3) (layers "F.Cu" "B.Cu") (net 3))
 (via (at 59.0804 53.3146) (size 0.6) (drill 0.3) (layers "F.Cu" "B.Cu") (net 3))
 (via (at 68.453 61.4934) (size 0.6) (drill 0.3) (layers "F.Cu" "B.Cu") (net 3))
 (segment (start 67.3862 61.4934) (end 68.453 61.4934) (width 0.25) (layer "B.Cu") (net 3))
 (segment (start 56.7182 54.8386) (end 58.2422 53.3146) (width 0.25) (layer "B.Cu") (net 3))
 (segment (start 60.6806 64.4398) (end 64.4398 64.4398) (width 0.25) (layer "B.Cu") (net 3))
 (segment (start 64.4398 64.4398) (end 67.3862 61.4934) (width 0.25) (layer "B.Cu") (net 3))
 (segment (start 56.7182 60.4774) (end 60.6806 64.4398) (width 0.25) (layer "B.Cu") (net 3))
 (segment (start 58.2422 53.3146) (end 59.0804 53.3146) (width 0.25) (layer "B.Cu") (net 3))
 (segment (start 56.7182 58.166) (end 56.7182 54.8386) (width 0.25) (layer "B.Cu") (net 3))
 (segment (start 56.7182 58.166) (end 56.7182 60.4774) (width 0.25) (layer "B.Cu") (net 3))
 (segment (start 60.6526 52.352) (end 60.8076 52.197) (width 0.25) (layer "F.Cu") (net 4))
 (segment (start 60.071 52.352) (end 60.6526 52.352) (width 0.25) (layer "F.Cu") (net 4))
 (segment (start 57.5564 53.1622) (end 58.3666 52.352) (width 0.25) (layer "F.Cu") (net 4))
 (segment (start 56.324 59.5) (end 57.5564 58.2676) (width 0.25) (layer "F.Cu") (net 4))
 (segment (start 64.8717 51.7397) (end 65.8622 51.7397) (width 0.25) (layer "F.Cu") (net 4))
 (segment (start 64.4144 52.197) (end 64.8717 51.7397) (width 0.25) (layer "F.Cu") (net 4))
 (segment (start 57.5564 56.3372) (end 57.5564 53.1622) (width 0.25) (layer "F.Cu") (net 4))
 (segment (start 57.5661 56.3275) (end 64.399584 56.3275) (width 0.25) (layer "F.Cu") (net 4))
 (segment (start 57.5564 58.2676) (end 57.5564 56.3372) (width 0.25) (layer "F.Cu") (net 4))
 (segment (start 63.627 52.197) (end 64.4144 52.197) (width 0.25) (layer "F.Cu") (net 4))
 (segment (start 57.5564 56.3372) (end 57.5661 56.3275) (width 0.25) (layer "F.Cu") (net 4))
 (segment (start 56.324 59.5) (end 54.98 59.5) (width 0.25) (layer "F.Cu") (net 4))
 (segment (start 58.3666 52.352) (end 60.071 52.352) (width 0.25) (layer "F.Cu") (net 4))
 (segment (start 64.399584 56.3275) (end 68.572084 60.5) (width 0.25) (layer "F.Cu") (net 4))
 (segment (start 68.572084 60.5) (end 70.42 60.5) (width 0.25) (layer "F.Cu") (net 4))
 (segment (start 61.727 52.197) (end 63.627 52.197) (width 0.25) (layer "F.Cu") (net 4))
 (segment (start 60.8076 52.197) (end 61.727 52.197) (width 0.25) (layer "F.Cu") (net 4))
 (segment (start 64.531 52.847) (end 63.627 52.847) (width 0.25) (layer "F.Cu") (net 10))
 (segment (start 65.8622 53.3147) (end 64.9987 53.3147) (width 0.25) (layer "F.Cu") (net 10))
 (segment (start 64.9987 53.3147) (end 64.531 52.847) (width 0.25) (layer "F.Cu") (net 10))
 (segment (start 57.24 61.5) (end 54.98 61.5) (width 0.25) (layer "F.Cu") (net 6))
 (segment (start 61.62 57.12) (end 57.24 61.5) (width 0.25) (layer "F.Cu") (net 6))
 (segment (start 68.453 58.49) (end 70.41 58.49) (width 0.25) (layer "F.Cu") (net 6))
 (segment (start 70.36 58.49) (end 70.37 58.5) (width 0.25) (layer "F.Cu") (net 6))
 (segment (start 70.41 58.49) (end 70.42 58.5) (width 0.25) (layer "F.Cu") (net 6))
 (segment (start 65.659 58.4708) (end 64.3082 57.12) (width 0.25) (layer "F.Cu") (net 6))
 (segment (start 70.31 58.49) (end 70.32 58.5) (width 0.25) (layer "F.Cu") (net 6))
 (segment (start 64.3082 57.12) (end 61.62 57.12) (width 0.25) (layer "F.Cu") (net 6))
 (via (at 68.453 58.49) (size 0.6) (drill 0.3) (layers "F.Cu" "B.Cu") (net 6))
 (via (at 65.659 58.4708) (size 0.6) (drill 0.3) (layers "F.Cu" "B.Cu") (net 6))
 (segment (start 68.453 58.49) (end 65.6782 58.49) (width 0.25) (layer "B.Cu") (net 6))
 (segment (start 65.6782 58.49) (end 65.659 58.4708) (width 0.25) (layer "B.Cu") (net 6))
 (segment (start 59.7916 57.2008) (end 59.7408 57.2008) (width 0.25) (layer "F.Cu") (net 5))
 (segment (start 68.472931 59.517669) (end 70.402331 59.517669) (width 0.25) (layer "F.Cu") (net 5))
 (segment (start 68.472931 59.517669) (end 68.4906 59.5) (width 0.25) (layer "F.Cu") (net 5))
 (segment (start 70.402331 59.517669) (end 70.42 59.5) (width 0.25) (layer "F.Cu") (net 5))
 (segment (start 59.7408 57.2008) (end 56.4416 60.5) (width 0.25) (layer "F.Cu") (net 5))
 (segment (start 56.4416 60.5) (end 54.98 60.5) (width 0.25) (layer "F.Cu") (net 5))
 (segment (start 68.472931 59.517669) (end 68.455262 59.5) (width 0.25) (layer "F.Cu") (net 5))
 (segment (start 70.352331 59.517669) (end 70.37 59.5) (width 0.25) (layer "F.Cu") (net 5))
 (via (at 59.7916 57.2008) (size 0.6) (drill 0.3) (layers "F.Cu" "B.Cu") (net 5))
 (via (at 68.472931 59.517669) (size 0.6) (drill 0.3) (layers "F.Cu" "B.Cu") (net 5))
 (segment (start 61.4492 57.2008) (end 59.7916 57.2008) (width 0.25) (layer "B.Cu") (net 5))
 (segment (start 68.472931 59.517669) (end 65.791469 59.517669) (width 0.25) (layer "B.Cu") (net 5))
 (segment (start 65.791469 59.517669) (end 63.4638 57.19) (width 0.25) (layer "B.Cu") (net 5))
 (segment (start 61.46 57.19) (end 61.4492 57.2008) (width 0.25) (layer "B.Cu") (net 5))
 (segment (start 63.4638 57.19) (end 61.46 57.19) (width 0.25) (layer "B.Cu") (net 5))
 (segment (start 63.627 54.4068) (end 63.1698 54.864) (width 0.25) (layer "F.Cu") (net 9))
 (segment (start 64.5202 65.881) (end 64.5202 66.081) (width 0.25) (layer "F.Cu") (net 9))
 (segment (start 62.8402 65.941) (end 62.8452 65.936) (width 0.25) (layer "F.Cu") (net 9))
 (segment (start 63.5452 65.936) (end 64.4652 65.936) (width 0.25) (layer "F.Cu") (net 9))
 (segment (start 61.6202 65.941) (end 60.4038 65.941) (width 0.25) (layer "F.Cu") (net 9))
 (segment (start 65.6082 68.5546) (end 65.1502 68.0966) (width 0.25) (layer "F.Cu") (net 9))
 (segment (start 58.55 65.1) (end 58.55 65.5858) (width 0.25) (layer "F.Cu") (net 9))
 (segment (start 62.8452 65.936) (end 63.5452 65.936) (width 0.25) (layer "F.Cu") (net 9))
 (segment (start 61.727 52.847) (end 62.1942 52.847) (width 0.25) (layer "F.Cu") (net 9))
 (segment (start 68.5546 68.5292) (end 65.6336 68.5292) (width 0.25) (layer "F.Cu") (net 9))
 (segment (start 65.1502 66.711) (end 65.1502 67.481) (width 0.25) (layer "F.Cu") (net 9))
 (segment (start 68.4754 54.6354) (end 68.83 54.99) (width 0.25) (layer "F.Cu") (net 9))
 (segment (start 63.627 53.497) (end 64.1396 53.497) (width 0.25) (layer "F.Cu") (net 9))
 (segment (start 65.278 54.6354) (end 68.4754 54.6354) (width 0.25) (layer "F.Cu") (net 9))
 (segment (start 62.1942 52.847) (end 62.8442 53.497) (width 0.25) (layer "F.Cu") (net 9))
 (segment (start 64.5202 66.081) (end 65.1502 66.711) (width 0.25) (layer "F.Cu") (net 9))
 (segment (start 61.6202 65.941) (end 62.8402 65.941) (width 0.25) (layer "F.Cu") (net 9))
 (segment (start 59.5628 65.1) (end 58.55 65.1) (width 0.25) (layer "F.Cu") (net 9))
 (segment (start 65.6336 68.5292) (end 65.6082 68.5546) (width 0.25) (layer "F.Cu") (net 9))
 (segment (start 63.627 53.497) (end 63.627 54.4068) (width 0.25) (layer "F.Cu") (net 9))
 (segment (start 64.1396 53.497) (end 65.278 54.6354) (width 0.25) (layer "F.Cu") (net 9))
 (segment (start 69.9008 67.183) (end 68.5546 68.5292) (width 0.25) (layer "F.Cu") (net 9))
 (segment (start 60.4038 65.941) (end 59.5628 65.1) (width 0.25) (layer "F.Cu") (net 9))
 (segment (start 69.9008 63.881) (end 69.9008 67.183) (width 0.25) (layer "F.Cu") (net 9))
 (segment (start 62.8442 53.497) (end 63.627 53.497) (width 0.25) (layer "F.Cu") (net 9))
 (segment (start 65.1502 68.0966) (end 65.1502 67.481) (width 0.25) (layer "F.Cu") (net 9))
 (segment (start 64.4652 65.936) (end 64.5202 65.881) (width 0.25) (layer "F.Cu") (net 9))
 (via (at 69.9008 63.881) (size 0.6) (drill 0.3) (layers "F.Cu" "B.Cu") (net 9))
 (via (at 68.83 54.99) (size 0.6) (drill 0.3) (layers "F.Cu" "B.Cu") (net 9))
 (segment (start 69.9008 56.0832) (end 68.83 55.0124) (width 0.25) (layer "B.Cu") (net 9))
 (segment (start 68.83 55.0124) (end 68.83 54.99) (width 0.25) (layer "B.Cu") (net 9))
 (segment (start 69.9008 63.881) (end 69.9008 56.0832) (width 0.25) (layer "B.Cu") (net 9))
 (segment (start 68.426 63.981) (end 68.4276 63.9826) (width 0.25) (layer "F.Cu") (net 1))
 (segment (start 66.802 61.9252) (end 66.802 63.3476) (width 0.25) (layer "F.Cu") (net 1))
 (segment (start 62.7 59.2125) (end 64.0893 59.2125) (width 0.25) (layer "F.Cu") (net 1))
 (segment (start 66.7952 63.981) (end 68.426 63.981) (width 0.25) (layer "F.Cu") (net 1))
 (segment (start 64.0893 59.2125) (end 66.802 61.9252) (width 0.25) (layer "F.Cu") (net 1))
 (segment (start 66.7952 63.3544) (end 66.7952 63.981) (width 0.25) (layer "F.Cu") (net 1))
 (segment (start 66.802 63.3476) (end 66.7952 63.3544) (width 0.25) (layer "F.Cu") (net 1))
 (segment (start 60.0375 60.7875) (end 62.7 60.7875) (width 0.25) (layer "F.Cu") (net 2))
 (segment (start 57.6 63.225) (end 57.6 62.56) (width 0.25) (layer "F.Cu") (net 2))
 (segment (start 57.6 63.225) (end 60.0375 60.7875) (width 0.25) (layer "F.Cu") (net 2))
 (segment (start 62.0058 63.225) (end 59.5 63.225) (width 0.25) (layer "F.Cu") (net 8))
 (segment (start 59.545 63.18) (end 59.5 63.225) (width 0.25) (layer "F.Cu") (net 8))
 (segment (start 64.5202 63.981) (end 62.7618 63.981) (width 0.25) (layer "F.Cu") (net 8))
 (segment (start 62.7618 63.981) (end 62.0058 63.225) (width 0.25) (layer "F.Cu") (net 8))
 (segment (start 66.7952 67.346) (end 66.6602 67.481) (width 0.25) (layer "F.Cu") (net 7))
 (segment (start 67.7164 67.3608) (end 68.4276 67.3608) (width 0.25) (layer "F.Cu") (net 7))
 (segment (start 66.7952 65.881) (end 66.7952 67.196) (width 0.25) (layer "F.Cu") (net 7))
 (segment (start 66.5226 67.481) (end 67.5962 67.481) (width 0.25) (layer "F.Cu") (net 7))
 (segment (start 66.5226 67.481) (end 66.1702 67.481) (width 0.25) (layer "F.Cu") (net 7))
 (segment (start 66.7952 67.196) (end 66.7952 67.346) (width 0.25) (layer "F.Cu") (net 7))
 (segment (start 66.6602 67.481) (end 66.5226 67.481) (width 0.25) (layer "F.Cu") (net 7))
 (segment (start 67.5962 67.481) (end 67.7164 67.3608) (width 0.25) (layer "F.Cu") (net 7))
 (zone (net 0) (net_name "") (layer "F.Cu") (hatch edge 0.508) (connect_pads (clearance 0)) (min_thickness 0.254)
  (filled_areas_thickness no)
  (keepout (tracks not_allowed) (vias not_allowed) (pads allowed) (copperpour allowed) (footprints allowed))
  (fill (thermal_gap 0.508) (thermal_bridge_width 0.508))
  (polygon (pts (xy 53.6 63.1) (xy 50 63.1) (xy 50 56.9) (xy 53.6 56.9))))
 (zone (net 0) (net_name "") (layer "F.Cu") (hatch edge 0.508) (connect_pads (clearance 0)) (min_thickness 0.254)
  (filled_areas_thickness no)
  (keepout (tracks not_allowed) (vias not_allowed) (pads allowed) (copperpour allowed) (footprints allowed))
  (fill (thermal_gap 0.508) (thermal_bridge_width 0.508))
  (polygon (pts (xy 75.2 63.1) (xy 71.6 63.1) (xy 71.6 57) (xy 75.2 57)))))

